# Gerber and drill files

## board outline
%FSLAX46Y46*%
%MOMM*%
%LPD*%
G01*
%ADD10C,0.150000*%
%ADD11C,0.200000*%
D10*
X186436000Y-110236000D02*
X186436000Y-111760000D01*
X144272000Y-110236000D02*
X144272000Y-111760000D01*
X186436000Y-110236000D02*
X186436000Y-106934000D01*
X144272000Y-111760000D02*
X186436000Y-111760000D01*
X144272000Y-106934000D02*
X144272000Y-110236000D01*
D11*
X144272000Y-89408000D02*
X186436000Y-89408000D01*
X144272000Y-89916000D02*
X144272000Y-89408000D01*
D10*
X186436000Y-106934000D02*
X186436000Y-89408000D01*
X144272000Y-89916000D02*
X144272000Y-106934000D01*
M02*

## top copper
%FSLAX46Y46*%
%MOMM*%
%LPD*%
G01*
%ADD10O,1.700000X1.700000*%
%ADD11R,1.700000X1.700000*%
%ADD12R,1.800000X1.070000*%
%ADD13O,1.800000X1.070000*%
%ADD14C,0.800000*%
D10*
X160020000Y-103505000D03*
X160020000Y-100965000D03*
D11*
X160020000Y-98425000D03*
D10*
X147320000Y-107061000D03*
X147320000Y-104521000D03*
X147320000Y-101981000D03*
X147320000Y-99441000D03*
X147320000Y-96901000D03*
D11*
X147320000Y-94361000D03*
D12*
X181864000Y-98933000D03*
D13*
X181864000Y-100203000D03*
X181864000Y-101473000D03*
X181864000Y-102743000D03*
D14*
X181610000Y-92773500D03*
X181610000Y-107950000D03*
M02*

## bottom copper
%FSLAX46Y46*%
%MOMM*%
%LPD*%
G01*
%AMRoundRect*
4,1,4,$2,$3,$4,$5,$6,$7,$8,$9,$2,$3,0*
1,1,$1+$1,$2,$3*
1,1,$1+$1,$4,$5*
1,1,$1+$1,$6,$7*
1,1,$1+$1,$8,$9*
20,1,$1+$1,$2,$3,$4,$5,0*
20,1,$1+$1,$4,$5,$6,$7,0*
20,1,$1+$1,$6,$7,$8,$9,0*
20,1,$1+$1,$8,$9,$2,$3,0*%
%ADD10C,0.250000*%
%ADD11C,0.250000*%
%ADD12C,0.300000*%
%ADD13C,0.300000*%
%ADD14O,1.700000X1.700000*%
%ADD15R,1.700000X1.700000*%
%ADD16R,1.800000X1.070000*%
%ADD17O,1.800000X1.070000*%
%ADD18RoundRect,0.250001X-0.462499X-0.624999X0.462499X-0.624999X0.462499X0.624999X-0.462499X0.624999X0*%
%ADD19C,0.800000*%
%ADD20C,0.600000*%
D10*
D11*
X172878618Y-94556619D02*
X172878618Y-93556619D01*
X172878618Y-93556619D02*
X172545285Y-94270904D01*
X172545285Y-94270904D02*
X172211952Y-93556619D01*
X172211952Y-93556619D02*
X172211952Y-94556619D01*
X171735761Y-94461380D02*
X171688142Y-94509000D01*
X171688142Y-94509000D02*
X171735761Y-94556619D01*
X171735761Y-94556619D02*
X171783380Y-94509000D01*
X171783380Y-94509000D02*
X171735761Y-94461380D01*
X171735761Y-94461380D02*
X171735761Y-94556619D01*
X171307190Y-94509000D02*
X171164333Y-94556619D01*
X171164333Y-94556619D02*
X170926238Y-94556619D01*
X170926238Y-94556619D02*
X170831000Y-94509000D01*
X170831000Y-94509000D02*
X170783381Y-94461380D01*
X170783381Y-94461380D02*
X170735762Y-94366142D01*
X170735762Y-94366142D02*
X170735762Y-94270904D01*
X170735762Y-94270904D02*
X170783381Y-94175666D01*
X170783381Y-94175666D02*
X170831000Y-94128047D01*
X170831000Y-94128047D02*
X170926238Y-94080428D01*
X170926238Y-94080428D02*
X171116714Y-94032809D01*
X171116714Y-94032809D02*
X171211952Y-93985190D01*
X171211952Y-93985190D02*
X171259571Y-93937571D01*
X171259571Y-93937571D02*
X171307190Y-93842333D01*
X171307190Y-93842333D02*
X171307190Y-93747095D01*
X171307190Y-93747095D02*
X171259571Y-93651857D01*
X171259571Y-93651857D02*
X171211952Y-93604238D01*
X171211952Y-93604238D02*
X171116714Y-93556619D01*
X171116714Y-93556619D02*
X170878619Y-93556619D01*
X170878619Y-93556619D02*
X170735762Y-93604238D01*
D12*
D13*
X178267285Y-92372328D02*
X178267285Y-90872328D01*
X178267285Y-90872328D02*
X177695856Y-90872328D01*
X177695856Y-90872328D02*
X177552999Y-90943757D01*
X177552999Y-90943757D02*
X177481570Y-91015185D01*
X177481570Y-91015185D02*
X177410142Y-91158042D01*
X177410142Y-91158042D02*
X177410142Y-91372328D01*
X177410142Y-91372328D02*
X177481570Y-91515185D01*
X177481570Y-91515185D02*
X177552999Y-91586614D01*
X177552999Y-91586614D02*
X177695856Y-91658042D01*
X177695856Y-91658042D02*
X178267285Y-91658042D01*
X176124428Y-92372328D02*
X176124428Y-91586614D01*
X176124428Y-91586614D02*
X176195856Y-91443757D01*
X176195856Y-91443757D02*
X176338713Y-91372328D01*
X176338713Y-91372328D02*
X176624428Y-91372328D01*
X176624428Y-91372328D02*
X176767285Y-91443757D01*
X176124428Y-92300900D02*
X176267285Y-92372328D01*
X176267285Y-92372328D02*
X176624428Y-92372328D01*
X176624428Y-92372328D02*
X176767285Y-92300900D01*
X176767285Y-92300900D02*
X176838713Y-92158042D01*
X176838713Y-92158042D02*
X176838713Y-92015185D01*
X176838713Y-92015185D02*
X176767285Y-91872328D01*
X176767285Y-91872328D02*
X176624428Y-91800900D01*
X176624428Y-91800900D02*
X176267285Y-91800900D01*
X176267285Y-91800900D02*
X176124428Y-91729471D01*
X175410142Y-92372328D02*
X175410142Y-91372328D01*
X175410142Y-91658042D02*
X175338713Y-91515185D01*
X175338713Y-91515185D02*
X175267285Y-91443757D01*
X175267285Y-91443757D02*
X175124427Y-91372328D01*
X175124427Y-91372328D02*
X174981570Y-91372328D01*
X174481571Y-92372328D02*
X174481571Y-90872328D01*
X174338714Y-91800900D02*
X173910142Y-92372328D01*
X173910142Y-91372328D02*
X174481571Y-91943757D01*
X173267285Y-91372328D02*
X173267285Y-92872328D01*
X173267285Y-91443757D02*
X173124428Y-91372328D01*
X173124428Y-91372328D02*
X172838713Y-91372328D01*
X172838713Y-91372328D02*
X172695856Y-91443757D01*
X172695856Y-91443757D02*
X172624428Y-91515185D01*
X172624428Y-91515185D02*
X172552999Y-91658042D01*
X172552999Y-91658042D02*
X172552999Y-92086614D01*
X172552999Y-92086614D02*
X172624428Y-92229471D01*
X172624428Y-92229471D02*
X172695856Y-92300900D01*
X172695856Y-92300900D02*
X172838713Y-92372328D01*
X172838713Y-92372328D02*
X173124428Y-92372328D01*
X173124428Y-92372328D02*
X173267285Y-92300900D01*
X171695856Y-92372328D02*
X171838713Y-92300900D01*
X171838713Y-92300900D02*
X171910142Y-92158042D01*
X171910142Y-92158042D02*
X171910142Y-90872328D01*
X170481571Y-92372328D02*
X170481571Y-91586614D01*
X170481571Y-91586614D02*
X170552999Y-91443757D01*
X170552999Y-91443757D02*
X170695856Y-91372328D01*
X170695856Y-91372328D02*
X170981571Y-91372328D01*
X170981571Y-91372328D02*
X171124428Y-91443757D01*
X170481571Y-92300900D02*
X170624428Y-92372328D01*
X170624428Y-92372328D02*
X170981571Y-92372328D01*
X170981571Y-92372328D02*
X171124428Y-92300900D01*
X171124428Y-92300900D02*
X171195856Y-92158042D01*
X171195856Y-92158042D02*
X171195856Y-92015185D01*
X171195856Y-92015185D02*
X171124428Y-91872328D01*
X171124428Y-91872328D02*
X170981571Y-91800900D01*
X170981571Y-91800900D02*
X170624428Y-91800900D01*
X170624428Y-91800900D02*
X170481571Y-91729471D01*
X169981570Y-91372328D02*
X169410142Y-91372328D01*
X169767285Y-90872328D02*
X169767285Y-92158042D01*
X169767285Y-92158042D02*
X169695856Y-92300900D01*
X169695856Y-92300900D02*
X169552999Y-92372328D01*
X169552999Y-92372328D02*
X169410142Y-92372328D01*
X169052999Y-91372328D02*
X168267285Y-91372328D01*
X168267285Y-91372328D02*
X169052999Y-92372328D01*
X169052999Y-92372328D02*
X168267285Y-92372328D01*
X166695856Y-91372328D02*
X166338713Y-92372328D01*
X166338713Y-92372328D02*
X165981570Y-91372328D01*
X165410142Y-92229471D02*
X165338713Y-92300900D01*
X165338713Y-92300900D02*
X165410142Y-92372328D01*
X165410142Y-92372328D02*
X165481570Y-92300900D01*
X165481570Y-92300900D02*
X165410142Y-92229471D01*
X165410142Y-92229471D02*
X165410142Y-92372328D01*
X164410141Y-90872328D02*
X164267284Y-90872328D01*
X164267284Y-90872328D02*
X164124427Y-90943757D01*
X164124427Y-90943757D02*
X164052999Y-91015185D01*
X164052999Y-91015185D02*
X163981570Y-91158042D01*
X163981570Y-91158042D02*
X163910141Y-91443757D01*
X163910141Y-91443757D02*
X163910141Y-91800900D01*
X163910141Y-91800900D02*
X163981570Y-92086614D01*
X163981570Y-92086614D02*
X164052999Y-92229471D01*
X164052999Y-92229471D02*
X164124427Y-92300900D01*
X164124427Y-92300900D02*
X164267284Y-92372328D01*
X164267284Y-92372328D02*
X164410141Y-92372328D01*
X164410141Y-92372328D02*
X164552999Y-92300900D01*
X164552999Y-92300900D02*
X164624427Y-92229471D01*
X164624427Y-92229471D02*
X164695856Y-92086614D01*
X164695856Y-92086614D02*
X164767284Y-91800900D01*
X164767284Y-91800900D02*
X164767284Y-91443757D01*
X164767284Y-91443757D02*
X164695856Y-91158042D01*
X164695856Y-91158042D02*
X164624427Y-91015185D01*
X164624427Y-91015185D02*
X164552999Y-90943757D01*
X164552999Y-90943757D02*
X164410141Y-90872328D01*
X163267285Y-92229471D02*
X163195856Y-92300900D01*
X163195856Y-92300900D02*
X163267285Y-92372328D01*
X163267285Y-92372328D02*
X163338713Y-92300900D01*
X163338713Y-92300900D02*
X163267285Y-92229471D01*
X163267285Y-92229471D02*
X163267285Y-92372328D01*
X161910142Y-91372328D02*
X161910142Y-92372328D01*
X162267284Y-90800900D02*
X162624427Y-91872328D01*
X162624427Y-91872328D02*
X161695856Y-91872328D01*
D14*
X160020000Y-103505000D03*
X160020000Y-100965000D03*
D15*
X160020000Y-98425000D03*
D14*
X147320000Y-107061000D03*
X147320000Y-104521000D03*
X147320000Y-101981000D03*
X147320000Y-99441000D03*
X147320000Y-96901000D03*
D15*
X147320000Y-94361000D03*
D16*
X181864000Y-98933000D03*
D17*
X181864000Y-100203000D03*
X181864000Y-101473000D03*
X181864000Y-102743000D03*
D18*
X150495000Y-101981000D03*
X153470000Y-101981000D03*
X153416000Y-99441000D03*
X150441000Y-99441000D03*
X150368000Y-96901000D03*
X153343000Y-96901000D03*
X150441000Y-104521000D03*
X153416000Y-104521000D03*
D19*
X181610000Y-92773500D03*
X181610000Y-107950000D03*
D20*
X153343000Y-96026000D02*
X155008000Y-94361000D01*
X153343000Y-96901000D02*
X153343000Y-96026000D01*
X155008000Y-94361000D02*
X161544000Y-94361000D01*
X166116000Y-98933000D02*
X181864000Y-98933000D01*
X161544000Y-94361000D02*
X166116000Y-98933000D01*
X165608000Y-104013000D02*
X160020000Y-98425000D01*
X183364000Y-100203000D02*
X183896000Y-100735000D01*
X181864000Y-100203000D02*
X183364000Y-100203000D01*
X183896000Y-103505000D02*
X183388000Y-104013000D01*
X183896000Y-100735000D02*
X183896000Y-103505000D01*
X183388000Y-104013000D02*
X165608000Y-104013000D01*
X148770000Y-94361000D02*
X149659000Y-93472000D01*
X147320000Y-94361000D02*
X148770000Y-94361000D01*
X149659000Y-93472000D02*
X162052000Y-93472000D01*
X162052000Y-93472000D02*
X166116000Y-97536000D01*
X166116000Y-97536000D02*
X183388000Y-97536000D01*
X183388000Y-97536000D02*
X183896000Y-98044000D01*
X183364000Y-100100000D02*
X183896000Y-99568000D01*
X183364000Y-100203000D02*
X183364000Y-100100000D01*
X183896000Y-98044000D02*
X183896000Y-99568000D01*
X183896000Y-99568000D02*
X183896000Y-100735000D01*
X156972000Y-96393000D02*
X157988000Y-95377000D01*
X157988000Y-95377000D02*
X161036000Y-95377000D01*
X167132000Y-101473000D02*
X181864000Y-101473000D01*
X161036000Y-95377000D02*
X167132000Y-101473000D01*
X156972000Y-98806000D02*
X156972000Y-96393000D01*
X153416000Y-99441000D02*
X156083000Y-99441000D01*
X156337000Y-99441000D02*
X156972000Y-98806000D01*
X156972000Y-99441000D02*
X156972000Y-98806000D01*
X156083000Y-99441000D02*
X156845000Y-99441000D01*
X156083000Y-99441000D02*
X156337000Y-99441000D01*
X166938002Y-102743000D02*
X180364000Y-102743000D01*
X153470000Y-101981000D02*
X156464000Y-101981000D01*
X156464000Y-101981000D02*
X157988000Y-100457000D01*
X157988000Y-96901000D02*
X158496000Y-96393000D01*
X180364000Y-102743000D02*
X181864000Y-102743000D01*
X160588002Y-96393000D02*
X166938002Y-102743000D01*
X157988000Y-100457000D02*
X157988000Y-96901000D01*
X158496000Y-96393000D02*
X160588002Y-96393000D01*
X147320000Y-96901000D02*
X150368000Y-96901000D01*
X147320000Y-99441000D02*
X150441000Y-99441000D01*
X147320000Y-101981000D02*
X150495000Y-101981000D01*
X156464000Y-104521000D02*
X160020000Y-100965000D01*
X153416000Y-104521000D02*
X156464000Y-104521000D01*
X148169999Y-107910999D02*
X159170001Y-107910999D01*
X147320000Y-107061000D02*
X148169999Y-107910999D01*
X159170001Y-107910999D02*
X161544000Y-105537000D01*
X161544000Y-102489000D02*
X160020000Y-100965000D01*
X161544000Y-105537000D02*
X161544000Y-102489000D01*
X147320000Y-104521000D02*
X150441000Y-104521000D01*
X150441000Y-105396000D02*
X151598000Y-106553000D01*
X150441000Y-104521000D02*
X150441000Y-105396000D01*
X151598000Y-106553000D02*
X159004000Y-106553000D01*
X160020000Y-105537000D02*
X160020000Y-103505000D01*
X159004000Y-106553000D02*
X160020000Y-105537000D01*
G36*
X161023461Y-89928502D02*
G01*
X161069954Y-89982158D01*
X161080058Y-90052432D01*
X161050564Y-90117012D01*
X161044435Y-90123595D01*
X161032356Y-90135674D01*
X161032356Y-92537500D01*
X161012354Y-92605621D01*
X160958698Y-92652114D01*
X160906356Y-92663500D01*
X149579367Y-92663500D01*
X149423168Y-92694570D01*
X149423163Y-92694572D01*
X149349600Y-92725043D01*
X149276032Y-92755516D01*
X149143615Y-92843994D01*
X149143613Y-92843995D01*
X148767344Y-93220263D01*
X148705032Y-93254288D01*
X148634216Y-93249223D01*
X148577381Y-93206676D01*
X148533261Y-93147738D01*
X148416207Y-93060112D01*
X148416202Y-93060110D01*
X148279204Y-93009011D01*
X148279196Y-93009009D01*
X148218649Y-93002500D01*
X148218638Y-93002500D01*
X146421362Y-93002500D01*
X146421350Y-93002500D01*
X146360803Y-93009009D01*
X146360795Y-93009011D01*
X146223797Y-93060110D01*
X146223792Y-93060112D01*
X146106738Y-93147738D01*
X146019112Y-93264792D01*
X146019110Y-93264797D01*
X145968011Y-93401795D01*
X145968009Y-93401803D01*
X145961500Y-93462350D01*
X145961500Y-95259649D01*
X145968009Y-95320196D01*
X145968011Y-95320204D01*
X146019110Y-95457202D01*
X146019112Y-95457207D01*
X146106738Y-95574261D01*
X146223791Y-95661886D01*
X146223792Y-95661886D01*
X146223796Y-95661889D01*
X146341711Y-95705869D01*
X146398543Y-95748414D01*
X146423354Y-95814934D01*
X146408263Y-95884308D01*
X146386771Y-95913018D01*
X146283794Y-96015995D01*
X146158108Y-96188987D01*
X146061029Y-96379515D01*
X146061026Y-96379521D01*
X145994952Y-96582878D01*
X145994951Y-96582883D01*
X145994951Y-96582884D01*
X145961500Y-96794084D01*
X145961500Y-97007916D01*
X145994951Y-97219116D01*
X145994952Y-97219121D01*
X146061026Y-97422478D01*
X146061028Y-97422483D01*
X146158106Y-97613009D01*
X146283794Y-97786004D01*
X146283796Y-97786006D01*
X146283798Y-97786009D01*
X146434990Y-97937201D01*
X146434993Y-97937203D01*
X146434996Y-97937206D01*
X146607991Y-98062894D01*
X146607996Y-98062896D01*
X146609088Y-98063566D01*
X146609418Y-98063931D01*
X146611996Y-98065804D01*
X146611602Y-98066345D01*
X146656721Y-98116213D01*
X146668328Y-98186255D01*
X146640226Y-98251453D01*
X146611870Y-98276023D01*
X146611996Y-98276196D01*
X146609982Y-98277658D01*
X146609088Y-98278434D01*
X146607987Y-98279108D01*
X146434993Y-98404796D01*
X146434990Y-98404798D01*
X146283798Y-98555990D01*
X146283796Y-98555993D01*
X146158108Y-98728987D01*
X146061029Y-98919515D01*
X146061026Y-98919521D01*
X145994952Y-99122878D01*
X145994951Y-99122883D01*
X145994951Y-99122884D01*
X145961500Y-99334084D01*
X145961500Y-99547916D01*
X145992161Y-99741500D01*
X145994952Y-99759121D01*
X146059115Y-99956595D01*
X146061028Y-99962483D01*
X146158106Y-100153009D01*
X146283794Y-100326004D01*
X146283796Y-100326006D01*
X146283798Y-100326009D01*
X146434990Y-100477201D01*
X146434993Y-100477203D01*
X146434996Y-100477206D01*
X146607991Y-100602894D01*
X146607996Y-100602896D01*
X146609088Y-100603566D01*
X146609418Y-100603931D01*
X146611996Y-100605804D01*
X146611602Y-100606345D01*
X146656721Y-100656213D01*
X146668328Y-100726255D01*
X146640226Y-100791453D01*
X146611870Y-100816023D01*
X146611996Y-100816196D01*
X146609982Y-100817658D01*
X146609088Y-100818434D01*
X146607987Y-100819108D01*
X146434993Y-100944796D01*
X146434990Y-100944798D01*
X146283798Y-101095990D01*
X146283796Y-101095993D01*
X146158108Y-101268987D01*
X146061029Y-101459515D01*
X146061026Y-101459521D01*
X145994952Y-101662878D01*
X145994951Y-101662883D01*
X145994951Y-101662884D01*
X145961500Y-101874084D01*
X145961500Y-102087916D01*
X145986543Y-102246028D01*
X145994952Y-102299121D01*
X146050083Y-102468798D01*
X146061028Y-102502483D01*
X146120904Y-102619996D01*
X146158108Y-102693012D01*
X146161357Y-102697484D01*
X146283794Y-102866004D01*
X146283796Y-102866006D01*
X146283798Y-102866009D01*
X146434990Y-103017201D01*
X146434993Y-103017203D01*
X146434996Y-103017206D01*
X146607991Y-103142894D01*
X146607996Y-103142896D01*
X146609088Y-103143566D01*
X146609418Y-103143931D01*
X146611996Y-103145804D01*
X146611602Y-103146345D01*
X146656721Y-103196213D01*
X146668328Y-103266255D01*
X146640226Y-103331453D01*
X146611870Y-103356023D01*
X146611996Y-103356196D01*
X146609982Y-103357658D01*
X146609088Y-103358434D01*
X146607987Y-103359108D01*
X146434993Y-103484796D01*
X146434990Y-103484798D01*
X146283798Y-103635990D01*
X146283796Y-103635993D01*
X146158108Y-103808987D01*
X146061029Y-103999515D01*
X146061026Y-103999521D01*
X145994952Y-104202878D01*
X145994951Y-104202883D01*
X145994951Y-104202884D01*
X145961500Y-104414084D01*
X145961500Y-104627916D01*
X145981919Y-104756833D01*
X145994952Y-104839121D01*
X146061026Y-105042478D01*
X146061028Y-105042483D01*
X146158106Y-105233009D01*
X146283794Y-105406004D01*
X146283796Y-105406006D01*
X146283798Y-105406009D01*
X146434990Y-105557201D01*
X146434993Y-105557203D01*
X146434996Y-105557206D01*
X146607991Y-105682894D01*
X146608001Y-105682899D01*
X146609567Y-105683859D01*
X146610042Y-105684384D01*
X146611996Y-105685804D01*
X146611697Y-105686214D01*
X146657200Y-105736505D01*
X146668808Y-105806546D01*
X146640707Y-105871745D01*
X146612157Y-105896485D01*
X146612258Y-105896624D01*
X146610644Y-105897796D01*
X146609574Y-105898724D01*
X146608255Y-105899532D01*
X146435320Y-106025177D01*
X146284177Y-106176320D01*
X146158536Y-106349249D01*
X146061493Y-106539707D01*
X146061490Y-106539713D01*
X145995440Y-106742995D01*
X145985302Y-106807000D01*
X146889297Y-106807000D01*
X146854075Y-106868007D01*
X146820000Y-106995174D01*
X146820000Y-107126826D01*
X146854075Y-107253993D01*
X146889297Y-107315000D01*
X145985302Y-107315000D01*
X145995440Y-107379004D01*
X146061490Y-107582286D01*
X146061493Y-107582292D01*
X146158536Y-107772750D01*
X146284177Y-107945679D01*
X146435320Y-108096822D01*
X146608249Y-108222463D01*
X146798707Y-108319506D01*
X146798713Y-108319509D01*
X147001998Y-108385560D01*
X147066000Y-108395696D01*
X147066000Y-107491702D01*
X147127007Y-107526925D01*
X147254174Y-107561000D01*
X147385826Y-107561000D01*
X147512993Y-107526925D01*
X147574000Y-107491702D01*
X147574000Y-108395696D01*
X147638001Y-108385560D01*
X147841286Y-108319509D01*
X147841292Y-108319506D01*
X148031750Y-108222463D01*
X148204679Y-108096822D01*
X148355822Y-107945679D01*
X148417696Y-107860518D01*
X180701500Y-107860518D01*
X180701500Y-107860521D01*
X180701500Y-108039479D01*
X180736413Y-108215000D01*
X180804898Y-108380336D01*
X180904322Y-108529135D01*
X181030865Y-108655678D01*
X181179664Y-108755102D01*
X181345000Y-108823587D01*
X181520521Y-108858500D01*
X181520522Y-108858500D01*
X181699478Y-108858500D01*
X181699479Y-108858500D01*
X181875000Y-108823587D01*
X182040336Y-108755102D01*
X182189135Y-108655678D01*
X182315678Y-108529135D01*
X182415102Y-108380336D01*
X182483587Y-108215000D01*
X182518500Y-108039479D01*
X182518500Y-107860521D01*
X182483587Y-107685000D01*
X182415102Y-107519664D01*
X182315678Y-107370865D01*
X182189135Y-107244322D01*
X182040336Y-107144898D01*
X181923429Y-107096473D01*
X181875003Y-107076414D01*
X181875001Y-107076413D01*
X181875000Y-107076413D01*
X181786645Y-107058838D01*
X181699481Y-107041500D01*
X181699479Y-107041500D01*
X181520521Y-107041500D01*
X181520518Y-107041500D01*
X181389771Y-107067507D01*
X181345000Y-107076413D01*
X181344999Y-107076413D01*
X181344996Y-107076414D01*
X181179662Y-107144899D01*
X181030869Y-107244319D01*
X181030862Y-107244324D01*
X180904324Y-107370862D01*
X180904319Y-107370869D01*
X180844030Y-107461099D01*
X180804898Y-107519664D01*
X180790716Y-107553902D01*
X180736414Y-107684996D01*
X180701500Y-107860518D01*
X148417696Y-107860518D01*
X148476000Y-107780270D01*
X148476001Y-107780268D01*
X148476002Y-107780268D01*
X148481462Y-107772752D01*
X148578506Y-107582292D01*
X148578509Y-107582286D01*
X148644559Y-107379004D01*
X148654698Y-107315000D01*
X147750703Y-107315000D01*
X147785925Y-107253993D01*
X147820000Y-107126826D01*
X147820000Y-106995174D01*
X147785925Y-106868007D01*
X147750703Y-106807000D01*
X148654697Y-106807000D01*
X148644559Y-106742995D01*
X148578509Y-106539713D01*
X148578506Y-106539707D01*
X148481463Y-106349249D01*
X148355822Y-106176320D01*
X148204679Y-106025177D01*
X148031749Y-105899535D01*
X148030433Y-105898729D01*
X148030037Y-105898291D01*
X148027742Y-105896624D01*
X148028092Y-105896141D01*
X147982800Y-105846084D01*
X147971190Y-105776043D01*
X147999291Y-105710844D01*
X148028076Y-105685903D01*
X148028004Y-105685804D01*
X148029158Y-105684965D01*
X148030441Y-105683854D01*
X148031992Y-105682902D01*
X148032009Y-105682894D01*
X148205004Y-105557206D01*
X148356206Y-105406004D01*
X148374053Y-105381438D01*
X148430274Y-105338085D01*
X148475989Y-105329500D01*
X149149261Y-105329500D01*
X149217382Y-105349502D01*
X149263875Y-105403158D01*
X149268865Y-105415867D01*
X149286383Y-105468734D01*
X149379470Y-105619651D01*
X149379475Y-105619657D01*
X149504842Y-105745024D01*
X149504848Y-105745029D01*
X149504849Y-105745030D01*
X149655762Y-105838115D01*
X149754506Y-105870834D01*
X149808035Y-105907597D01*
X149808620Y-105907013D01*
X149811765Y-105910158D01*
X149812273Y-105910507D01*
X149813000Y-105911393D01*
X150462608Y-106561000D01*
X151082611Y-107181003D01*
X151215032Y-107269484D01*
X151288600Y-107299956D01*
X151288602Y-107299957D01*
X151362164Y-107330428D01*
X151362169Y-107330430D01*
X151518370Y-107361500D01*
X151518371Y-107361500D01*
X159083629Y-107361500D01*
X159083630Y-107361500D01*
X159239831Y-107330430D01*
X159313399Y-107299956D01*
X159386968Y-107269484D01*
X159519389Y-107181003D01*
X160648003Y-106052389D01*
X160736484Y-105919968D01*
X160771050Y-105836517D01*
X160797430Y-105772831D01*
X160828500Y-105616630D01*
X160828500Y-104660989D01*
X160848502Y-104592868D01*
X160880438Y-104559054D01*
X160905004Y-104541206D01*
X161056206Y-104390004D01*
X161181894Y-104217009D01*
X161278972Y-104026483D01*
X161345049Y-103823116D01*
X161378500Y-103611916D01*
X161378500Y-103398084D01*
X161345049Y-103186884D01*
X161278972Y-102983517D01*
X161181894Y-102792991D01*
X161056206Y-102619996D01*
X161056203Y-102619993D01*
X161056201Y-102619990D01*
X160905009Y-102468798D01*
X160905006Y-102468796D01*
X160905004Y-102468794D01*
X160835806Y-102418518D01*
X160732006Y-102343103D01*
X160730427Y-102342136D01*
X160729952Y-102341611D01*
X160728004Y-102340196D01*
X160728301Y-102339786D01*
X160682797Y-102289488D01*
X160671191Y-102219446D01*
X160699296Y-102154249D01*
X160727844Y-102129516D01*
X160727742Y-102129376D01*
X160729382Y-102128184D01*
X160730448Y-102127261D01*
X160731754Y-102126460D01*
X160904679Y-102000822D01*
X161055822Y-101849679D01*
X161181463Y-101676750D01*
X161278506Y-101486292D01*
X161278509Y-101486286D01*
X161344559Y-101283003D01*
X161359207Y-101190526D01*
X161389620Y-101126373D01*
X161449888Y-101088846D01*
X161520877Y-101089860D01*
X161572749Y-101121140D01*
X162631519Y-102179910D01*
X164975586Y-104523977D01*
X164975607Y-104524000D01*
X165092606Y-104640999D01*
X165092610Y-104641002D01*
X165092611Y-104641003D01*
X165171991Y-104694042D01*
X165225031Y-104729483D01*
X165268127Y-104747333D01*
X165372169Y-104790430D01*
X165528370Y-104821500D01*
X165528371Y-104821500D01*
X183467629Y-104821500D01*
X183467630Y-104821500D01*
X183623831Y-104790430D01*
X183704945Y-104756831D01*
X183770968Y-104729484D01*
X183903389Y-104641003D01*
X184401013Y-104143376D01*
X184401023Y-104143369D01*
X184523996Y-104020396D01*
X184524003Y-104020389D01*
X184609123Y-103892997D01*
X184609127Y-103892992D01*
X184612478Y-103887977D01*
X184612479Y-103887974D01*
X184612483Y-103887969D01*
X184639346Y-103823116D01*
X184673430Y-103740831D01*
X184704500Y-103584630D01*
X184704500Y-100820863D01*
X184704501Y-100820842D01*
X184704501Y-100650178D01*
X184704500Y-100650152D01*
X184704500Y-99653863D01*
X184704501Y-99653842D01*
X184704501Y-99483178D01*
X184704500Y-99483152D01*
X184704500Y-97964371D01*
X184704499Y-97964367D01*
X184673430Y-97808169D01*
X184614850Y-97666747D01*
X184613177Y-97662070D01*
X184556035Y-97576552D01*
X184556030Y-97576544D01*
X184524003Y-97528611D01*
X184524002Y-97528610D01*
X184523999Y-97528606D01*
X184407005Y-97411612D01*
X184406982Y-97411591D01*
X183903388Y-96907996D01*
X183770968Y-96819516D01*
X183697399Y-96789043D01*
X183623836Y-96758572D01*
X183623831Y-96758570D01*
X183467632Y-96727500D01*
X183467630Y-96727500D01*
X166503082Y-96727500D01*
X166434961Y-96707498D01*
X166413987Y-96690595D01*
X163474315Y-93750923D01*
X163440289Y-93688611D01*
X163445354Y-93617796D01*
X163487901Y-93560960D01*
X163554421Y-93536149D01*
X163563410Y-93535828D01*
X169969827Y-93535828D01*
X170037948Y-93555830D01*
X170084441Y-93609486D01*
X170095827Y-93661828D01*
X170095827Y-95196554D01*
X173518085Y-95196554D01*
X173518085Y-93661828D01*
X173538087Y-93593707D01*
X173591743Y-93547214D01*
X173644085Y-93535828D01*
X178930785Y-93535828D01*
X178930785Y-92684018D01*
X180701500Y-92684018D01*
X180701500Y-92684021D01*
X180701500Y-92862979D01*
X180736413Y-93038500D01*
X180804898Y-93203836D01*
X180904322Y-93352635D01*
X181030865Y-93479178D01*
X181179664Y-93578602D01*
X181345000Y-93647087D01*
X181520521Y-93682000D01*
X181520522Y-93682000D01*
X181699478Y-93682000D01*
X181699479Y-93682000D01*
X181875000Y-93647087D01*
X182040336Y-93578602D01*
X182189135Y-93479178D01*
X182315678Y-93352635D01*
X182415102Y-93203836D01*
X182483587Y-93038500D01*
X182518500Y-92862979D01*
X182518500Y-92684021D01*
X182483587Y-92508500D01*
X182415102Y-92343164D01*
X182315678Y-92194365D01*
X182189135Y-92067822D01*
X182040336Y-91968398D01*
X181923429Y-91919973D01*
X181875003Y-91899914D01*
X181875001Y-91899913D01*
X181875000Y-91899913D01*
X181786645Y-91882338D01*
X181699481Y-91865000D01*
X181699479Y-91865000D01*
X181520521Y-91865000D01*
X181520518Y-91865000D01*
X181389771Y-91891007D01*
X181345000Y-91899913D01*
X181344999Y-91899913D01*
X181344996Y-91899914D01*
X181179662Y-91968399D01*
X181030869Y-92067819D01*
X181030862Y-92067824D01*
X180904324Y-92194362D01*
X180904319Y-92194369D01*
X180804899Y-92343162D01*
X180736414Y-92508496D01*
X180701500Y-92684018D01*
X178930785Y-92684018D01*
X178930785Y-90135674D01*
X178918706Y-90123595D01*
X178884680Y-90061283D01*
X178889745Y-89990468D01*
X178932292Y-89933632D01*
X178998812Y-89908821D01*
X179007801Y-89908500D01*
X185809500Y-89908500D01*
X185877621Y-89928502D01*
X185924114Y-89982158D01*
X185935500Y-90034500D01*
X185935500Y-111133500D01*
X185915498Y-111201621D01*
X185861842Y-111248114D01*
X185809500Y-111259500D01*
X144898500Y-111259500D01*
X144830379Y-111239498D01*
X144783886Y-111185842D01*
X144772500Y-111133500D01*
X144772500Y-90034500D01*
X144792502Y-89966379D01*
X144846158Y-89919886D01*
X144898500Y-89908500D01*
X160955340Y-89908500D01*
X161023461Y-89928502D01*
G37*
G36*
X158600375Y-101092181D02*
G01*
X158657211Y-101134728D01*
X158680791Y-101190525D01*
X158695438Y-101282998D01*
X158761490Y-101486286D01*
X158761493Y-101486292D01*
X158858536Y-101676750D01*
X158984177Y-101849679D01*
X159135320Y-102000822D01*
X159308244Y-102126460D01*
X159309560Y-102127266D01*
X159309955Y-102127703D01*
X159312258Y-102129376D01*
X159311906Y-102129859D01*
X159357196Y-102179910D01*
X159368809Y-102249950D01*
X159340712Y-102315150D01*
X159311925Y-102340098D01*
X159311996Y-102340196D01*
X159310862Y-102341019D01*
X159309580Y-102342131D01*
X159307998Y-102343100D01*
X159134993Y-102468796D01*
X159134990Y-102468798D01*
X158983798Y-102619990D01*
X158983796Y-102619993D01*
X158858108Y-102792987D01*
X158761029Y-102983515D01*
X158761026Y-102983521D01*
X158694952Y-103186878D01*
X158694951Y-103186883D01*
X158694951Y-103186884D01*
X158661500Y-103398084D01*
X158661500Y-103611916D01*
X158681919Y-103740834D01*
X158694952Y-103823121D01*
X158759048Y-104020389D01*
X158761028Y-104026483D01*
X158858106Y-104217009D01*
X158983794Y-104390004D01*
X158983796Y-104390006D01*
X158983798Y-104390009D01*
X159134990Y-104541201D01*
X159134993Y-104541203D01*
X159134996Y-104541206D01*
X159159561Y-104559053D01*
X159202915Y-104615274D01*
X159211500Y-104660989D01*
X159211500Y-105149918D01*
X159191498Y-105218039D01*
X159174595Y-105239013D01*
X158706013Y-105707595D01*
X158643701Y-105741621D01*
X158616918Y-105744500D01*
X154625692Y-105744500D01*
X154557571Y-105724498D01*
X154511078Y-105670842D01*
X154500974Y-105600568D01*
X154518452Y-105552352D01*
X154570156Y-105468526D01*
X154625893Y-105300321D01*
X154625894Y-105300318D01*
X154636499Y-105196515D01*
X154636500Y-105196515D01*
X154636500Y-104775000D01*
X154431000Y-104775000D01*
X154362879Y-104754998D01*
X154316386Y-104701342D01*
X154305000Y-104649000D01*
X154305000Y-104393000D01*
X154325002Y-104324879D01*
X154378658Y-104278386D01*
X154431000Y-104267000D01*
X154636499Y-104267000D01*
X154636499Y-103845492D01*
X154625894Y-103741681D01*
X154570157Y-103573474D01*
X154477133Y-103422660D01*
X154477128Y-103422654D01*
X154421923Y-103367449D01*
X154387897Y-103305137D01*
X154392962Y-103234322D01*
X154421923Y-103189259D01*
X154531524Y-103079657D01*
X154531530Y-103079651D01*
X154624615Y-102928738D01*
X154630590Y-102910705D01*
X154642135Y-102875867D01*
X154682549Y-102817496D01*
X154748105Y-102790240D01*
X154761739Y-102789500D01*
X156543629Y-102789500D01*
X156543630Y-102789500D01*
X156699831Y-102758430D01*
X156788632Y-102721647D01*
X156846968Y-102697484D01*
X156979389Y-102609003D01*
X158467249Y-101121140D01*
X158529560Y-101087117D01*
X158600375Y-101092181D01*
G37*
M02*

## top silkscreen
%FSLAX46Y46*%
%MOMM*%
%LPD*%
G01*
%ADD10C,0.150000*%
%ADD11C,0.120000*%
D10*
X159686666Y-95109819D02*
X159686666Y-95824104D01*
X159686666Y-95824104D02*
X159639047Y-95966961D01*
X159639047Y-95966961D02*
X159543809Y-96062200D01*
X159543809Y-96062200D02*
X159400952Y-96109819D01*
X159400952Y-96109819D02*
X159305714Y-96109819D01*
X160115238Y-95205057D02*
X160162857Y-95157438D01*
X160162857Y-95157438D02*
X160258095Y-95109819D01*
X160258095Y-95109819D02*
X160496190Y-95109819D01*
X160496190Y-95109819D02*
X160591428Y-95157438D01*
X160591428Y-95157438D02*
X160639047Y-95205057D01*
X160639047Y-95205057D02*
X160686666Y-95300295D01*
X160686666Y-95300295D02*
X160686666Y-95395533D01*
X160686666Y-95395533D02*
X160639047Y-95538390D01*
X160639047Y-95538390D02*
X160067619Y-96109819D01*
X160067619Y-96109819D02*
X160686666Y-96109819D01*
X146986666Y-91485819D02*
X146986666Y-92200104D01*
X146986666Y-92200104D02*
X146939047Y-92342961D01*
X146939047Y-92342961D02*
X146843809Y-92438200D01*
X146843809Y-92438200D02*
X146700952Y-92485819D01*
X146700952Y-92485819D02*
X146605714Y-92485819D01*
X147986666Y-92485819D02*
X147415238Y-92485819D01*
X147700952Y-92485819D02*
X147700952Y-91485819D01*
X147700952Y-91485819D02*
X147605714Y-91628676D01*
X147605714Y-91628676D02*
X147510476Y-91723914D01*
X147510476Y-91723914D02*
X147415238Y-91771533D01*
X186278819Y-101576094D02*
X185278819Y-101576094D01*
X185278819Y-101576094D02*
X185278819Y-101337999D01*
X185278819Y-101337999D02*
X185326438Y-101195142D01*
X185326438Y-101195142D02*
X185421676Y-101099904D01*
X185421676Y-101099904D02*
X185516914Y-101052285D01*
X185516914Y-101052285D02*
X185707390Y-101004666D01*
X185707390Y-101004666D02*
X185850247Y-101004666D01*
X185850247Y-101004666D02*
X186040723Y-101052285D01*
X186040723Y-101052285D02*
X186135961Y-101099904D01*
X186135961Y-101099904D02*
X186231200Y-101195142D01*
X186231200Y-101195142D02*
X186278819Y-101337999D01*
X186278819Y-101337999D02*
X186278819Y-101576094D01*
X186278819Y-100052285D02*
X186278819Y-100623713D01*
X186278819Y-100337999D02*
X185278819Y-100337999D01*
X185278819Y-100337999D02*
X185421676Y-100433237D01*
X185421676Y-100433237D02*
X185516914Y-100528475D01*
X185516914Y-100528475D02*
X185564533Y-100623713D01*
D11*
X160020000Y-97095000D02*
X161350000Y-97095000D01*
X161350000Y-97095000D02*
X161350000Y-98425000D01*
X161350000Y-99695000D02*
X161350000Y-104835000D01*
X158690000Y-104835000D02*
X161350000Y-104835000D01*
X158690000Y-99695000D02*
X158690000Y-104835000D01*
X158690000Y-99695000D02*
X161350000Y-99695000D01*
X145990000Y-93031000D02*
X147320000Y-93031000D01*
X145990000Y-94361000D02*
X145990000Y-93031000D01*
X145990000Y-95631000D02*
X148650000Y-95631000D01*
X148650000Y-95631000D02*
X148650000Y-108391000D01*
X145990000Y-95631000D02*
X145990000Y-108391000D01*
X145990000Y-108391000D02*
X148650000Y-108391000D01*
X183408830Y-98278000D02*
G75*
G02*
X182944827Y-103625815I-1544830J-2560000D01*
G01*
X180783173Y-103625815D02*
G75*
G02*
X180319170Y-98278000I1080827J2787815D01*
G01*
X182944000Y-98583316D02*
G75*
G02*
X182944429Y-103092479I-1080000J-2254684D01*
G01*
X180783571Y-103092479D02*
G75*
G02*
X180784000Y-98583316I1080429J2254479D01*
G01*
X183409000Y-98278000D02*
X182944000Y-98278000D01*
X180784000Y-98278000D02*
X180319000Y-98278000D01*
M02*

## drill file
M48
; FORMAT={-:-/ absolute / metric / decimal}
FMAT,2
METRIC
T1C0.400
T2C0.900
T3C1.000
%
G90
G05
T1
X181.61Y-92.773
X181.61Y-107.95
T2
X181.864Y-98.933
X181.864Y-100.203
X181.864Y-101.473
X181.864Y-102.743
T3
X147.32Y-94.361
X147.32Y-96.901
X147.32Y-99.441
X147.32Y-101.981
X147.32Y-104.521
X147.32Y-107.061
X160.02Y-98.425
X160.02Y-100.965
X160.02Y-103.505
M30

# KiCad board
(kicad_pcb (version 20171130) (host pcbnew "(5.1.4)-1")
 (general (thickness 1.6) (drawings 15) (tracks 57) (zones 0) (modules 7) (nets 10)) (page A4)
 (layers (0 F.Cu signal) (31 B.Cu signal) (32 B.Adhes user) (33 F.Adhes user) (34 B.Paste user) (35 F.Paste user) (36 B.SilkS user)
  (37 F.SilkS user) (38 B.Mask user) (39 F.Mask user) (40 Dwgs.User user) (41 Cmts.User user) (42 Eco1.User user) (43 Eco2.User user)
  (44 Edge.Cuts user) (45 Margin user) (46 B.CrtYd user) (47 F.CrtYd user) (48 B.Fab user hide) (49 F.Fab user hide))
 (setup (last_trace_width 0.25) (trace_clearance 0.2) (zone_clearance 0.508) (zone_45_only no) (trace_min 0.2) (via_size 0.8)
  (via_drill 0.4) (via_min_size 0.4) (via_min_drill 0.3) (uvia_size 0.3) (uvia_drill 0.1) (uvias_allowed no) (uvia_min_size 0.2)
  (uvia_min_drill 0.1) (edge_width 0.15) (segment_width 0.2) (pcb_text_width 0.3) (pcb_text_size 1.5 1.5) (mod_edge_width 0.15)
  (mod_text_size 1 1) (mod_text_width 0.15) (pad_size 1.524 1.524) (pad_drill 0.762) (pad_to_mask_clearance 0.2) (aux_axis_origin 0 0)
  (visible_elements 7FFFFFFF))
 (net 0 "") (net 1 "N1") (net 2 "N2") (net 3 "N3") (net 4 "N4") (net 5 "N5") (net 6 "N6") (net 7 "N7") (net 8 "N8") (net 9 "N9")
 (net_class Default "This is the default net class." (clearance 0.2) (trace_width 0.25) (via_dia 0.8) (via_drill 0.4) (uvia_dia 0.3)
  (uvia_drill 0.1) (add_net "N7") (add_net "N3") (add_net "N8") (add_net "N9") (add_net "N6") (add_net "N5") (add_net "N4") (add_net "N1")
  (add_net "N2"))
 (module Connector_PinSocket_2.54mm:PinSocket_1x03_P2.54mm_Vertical (layer F.Cu) (at 160.02 98.425)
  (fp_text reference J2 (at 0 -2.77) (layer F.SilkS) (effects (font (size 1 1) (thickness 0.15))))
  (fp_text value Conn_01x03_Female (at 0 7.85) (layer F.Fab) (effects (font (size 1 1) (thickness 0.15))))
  (fp_line (start 0 -1.33) (end 1.33 -1.33) (layer F.SilkS) (width 0.12))
  (fp_line (start 1.33 -1.33) (end 1.33 0) (layer F.SilkS) (width 0.12))
  (fp_line (start 1.33 1.27) (end 1.33 6.41) (layer F.SilkS) (width 0.12))
  (fp_line (start -1.33 6.41) (end 1.33 6.41) (layer F.SilkS) (width 0.12))
  (fp_line (start -1.33 1.27) (end -1.33 6.41) (layer F.SilkS) (width 0.12))
  (fp_line (start -1.33 1.27) (end 1.33 1.27) (layer F.SilkS) (width 0.12))
  (pad 3 thru_hole oval (at 0 5.08) (size 1.7 1.7) (drill 1) (layers *.Cu *.Mask) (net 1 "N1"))
  (pad 2 thru_hole oval (at 0 2.54) (size 1.7 1.7) (drill 1) (layers *.Cu *.Mask) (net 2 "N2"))
  (pad 1 thru_hole rect (at 0 0) (size 1.7 1.7) (drill 1) (layers *.Cu *.Mask) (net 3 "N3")))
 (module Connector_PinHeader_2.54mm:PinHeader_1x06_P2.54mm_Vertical (layer F.Cu) (at 147.32 94.361)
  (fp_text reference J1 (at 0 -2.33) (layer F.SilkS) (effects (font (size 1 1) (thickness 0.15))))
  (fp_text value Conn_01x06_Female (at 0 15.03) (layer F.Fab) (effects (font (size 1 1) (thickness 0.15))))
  (fp_line (start -1.33 -1.33) (end 0 -1.33) (layer F.SilkS) (width 0.12))
  (fp_line (start -1.33 0) (end -1.33 -1.33) (layer F.SilkS) (width 0.12))
  (fp_line (start -1.33 1.27) (end 1.33 1.27) (layer F.SilkS) (width 0.12))
  (fp_line (start 1.33 1.27) (end 1.33 14.03) (layer F.SilkS) (width 0.12))
  (fp_line (start -1.33 1.27) (end -1.33 14.03) (layer F.SilkS) (width 0.12))
  (fp_line (start -1.33 14.03) (end 1.33 14.03) (layer F.SilkS) (width 0.12))
  (pad 6 thru_hole oval (at 0 12.7) (size 1.7 1.7) (drill 1) (layers *.Cu *.Mask) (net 2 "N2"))
  (pad 5 thru_hole oval (at 0 10.16) (size 1.7 1.7) (drill 1) (layers *.Cu *.Mask) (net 1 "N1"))
  (pad 4 thru_hole oval (at 0 7.62) (size 1.7 1.7) (drill 1) (layers *.Cu *.Mask) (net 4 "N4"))
  (pad 3 thru_hole oval (at 0 5.08) (size 1.7 1.7) (drill 1) (layers *.Cu *.Mask) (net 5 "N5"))
  (pad 2 thru_hole oval (at 0 2.54) (size 1.7 1.7) (drill 1) (layers *.Cu *.Mask) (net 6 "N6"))
  (pad 1 thru_hole rect (at 0 0) (size 1.7 1.7) (drill 1) (layers *.Cu *.Mask) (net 3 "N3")))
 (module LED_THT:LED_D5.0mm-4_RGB (layer F.Cu) (at 181.864 98.933 270)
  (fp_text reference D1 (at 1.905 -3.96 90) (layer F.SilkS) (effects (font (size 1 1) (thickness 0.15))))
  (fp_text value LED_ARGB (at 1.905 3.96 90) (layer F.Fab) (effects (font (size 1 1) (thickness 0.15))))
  (fp_arc (start 1.905 0) (end -0.655 -1.54483) (angle 127.7) (layer F.SilkS) (width 0.12))
  (fp_arc (start 1.905 0) (end -0.655 1.54483) (angle -127.7) (layer F.SilkS) (width 0.12))
  (fp_arc (start 1.905 0) (end -0.349684 -1.08) (angle 128.8) (layer F.SilkS) (width 0.12))
  (fp_arc (start 1.905 0) (end -0.349684 1.08) (angle -128.8) (layer F.SilkS) (width 0.12))
  (fp_line (start -0.655 -1.545) (end -0.655 -1.08) (layer F.SilkS) (width 0.12))
  (fp_line (start -0.655 1.08) (end -0.655 1.545) (layer F.SilkS) (width 0.12))
  (pad 1 thru_hole rect (at 0 0 270) (size 1.07 1.8) (drill 0.9) (layers *.Cu *.Mask) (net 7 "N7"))
  (pad 2 thru_hole oval (at 1.27 0 270) (size 1.07 1.8) (drill 0.9) (layers *.Cu *.Mask) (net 3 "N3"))
  (pad 3 thru_hole oval (at 2.54 0 270) (size 1.07 1.8) (drill 0.9) (layers *.Cu *.Mask) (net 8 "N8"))
  (pad 4 thru_hole oval (at 3.81 0 270) (size 1.07 1.8) (drill 0.9) (layers *.Cu *.Mask) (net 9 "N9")))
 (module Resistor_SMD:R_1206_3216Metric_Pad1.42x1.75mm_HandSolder (layer B.Cu) (at 151.9825 101.981)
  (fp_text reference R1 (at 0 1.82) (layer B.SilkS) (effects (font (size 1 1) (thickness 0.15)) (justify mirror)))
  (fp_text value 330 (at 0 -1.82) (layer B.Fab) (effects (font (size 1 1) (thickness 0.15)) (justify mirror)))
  (pad 1 smd roundrect (at -1.4875 0) (size 1.425 1.75) (layers B.Cu B.Paste B.Mask) (roundrect_rratio 0.175439) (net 4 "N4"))
  (pad 2 smd roundrect (at 1.4875 0) (size 1.425 1.75) (layers B.Cu B.Paste B.Mask) (roundrect_rratio 0.175439) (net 9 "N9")))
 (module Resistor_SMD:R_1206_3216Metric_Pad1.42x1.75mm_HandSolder (layer B.Cu) (at 151.9285 99.441)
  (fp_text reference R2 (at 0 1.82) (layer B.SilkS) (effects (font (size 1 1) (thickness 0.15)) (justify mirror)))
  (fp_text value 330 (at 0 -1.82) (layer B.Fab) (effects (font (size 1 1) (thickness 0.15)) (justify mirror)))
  (pad 2 smd roundrect (at 1.4875 0) (size 1.425 1.75) (layers B.Cu B.Paste B.Mask) (roundrect_rratio 0.175439) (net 8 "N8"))
  (pad 1 smd roundrect (at -1.4875 0) (size 1.425 1.75) (layers B.Cu B.Paste B.Mask) (roundrect_rratio 0.175439) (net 5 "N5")))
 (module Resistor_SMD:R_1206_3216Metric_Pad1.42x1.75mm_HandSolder (layer B.Cu) (at 151.8555 96.901)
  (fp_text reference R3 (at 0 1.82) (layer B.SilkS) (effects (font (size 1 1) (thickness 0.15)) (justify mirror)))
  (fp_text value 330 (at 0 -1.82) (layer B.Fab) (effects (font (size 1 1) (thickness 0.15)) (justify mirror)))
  (pad 1 smd roundrect (at -1.4875 0) (size 1.425 1.75) (layers B.Cu B.Paste B.Mask) (roundrect_rratio 0.175439) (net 6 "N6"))
  (pad 2 smd roundrect (at 1.4875 0) (size 1.425 1.75) (layers B.Cu B.Paste B.Mask) (roundrect_rratio 0.175439) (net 7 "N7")))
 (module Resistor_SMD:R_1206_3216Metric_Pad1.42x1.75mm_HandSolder (layer B.Cu) (at 151.9285 104.521)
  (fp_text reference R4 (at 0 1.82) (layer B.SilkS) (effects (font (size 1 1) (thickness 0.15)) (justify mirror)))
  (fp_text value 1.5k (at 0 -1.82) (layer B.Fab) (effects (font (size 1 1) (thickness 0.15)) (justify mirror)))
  (pad 1 smd roundrect (at -1.4875 0) (size 1.425 1.75) (layers B.Cu B.Paste B.Mask) (roundrect_rratio 0.175439) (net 1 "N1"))
  (pad 2 smd roundrect (at 1.4875 0) (size 1.425 1.75) (layers B.Cu B.Paste B.Mask) (roundrect_rratio 0.175439) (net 2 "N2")))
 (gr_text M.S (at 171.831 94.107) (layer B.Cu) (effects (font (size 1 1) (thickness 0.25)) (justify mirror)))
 (gr_line (start 186.436 110.236) (end 186.436 111.76) (layer Edge.Cuts) (width 0.15))
 (gr_line (start 144.272 110.236) (end 144.272 111.76) (layer Edge.Cuts) (width 0.15))
 (gr_line (start 186.436 110.236) (end 186.436 106.934) (layer Edge.Cuts) (width 0.15))
 (gr_line (start 144.272 111.76) (end 186.436 111.76) (layer Edge.Cuts) (width 0.15))
 (gr_line (start 144.272 106.934) (end 144.272 110.236) (layer Edge.Cuts) (width 0.15))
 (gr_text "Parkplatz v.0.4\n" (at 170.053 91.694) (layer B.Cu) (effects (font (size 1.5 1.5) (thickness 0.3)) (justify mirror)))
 (gr_line (start 144.272 89.408) (end 186.436 89.408) (layer Edge.Cuts) (width 0.2))
 (gr_line (start 144.272 89.916) (end 144.272 89.408) (layer Edge.Cuts) (width 0.2))
 (gr_line (start 186.436 106.934) (end 186.436 89.408) (layer Edge.Cuts) (width 0.15))
 (gr_line (start 144.272 89.916) (end 144.272 106.934) (layer Edge.Cuts) (width 0.15))
 (via (at 181.61 92.7735) (size 0.8) (drill 0.4) (layers F.Cu B.Cu) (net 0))
 (via (at 181.61 107.95) (size 0.8) (drill 0.4) (layers F.Cu B.Cu) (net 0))
 (segment (start 153.343 96.026) (end 155.008 94.361) (width 0.6) (layer B.Cu) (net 7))
 (segment (start 153.343 96.901) (end 153.343 96.026) (width 0.6) (layer B.Cu) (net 7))
 (segment (start 155.008 94.361) (end 161.544 94.361) (width 0.6) (layer B.Cu) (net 7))
 (segment (start 166.116 98.933) (end 181.864 98.933) (width 0.6) (layer B.Cu) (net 7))
 (segment (start 161.544 94.361) (end 166.116 98.933) (width 0.6) (layer B.Cu) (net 7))
 (segment (start 165.608 104.013) (end 160.02 98.425) (width 0.6) (layer B.Cu) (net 3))
 (segment (start 183.364 100.203) (end 183.896 100.735) (width 0.6) (layer B.Cu) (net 3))
 (segment (start 181.864 100.203) (end 183.364 100.203) (width 0.6) (layer B.Cu) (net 3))
 (segment (start 183.896 103.505) (end 183.388 104.013) (width 0.6) (layer B.Cu) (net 3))
 (segment (start 183.896 100.735) (end 183.896 103.505) (width 0.6) (layer B.Cu) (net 3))
 (segment (start 183.388 104.013) (end 165.608 104.013) (width 0.6) (layer B.Cu) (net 3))
 (segment (start 148.77 94.361) (end 149.659 93.472) (width 0.6) (layer B.Cu) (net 3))
 (segment (start 147.32 94.361) (end 148.77 94.361) (width 0.6) (layer B.Cu) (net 3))
 (segment (start 149.659 93.472) (end 162.052 93.472) (width 0.6) (layer B.Cu) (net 3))
 (segment (start 162.052 93.472) (end 166.116 97.536) (width 0.6) (layer B.Cu) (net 3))
 (segment (start 166.116 97.536) (end 183.388 97.536) (width 0.6) (layer B.Cu) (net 3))
 (segment (start 183.388 97.536) (end 183.896 98.044) (width 0.6) (layer B.Cu) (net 3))
 (segment (start 183.364 100.1) (end 183.896 99.568) (width 0.6) (layer B.Cu) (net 3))
 (segment (start 183.364 100.203) (end 183.364 100.1) (width 0.6) (layer B.Cu) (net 3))
 (segment (start 183.896 98.044) (end 183.896 99.568) (width 0.6) (layer B.Cu) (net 3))
 (segment (start 183.896 99.568) (end 183.896 100.735) (width 0.6) (layer B.Cu) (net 3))
 (segment (start 156.972 96.393) (end 157.988 95.377) (width 0.6) (layer B.Cu) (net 8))
 (segment (start 157.988 95.377) (end 161.036 95.377) (width 0.6) (layer B.Cu) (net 8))
 (segment (start 167.132 101.473) (end 181.864 101.473) (width 0.6) (layer B.Cu) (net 8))
 (segment (start 161.036 95.377) (end 167.132 101.473) (width 0.6) (layer B.Cu) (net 8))
 (segment (start 156.972 98.806) (end 156.972 96.393) (width 0.6) (layer B.Cu) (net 8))
 (segment (start 153.416 99.441) (end 156.083 99.441) (width 0.6) (layer B.Cu) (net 8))
 (segment (start 156.337 99.441) (end 156.972 98.806) (width 0.6) (layer B.Cu) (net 8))
 (segment (start 156.972 99.441) (end 156.972 98.806) (width 0.6) (layer B.Cu) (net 8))
 (segment (start 156.083 99.441) (end 156.845 99.441) (width 0.6) (layer B.Cu) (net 8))
 (segment (start 156.083 99.441) (end 156.337 99.441) (width 0.6) (layer B.Cu) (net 8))
 (segment (start 166.938002 102.743) (end 180.364 102.743) (width 0.6) (layer B.Cu) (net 9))
 (segment (start 153.47 101.981) (end 156.464 101.981) (width 0.6) (layer B.Cu) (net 9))
 (segment (start 156.464 101.981) (end 157.988 100.457) (width 0.6) (layer B.Cu) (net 9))
 (segment (start 157.988 96.901) (end 158.496 96.393) (width 0.6) (layer B.Cu) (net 9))
 (segment (start 180.364 102.743) (end 181.864 102.743) (width 0.6) (layer B.Cu) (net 9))
 (segment (start 160.588002 96.393) (end 166.938002 102.743) (width 0.6) (layer B.Cu) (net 9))
 (segment (start 157.988 100.457) (end 157.988 96.901) (width 0.6) (layer B.Cu) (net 9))
 (segment (start 158.496 96.393) (end 160.588002 96.393) (width 0.6) (layer B.Cu) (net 9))
 (segment (start 147.32 96.901) (end 150.368 96.901) (width 0.6) (layer B.Cu) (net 6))
 (segment (start 147.32 99.441) (end 150.441 99.441) (width 0.6) (layer B.Cu) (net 5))
 (segment (start 147.32 101.981) (end 150.495 101.981) (width 0.6) (layer B.Cu) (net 4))
 (segment (start 156.464 104.521) (end 160.02 100.965) (width 0.6) (layer B.Cu) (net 2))
 (segment (start 153.416 104.521) (end 156.464 104.521) (width 0.6) (layer B.Cu) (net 2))
 (segment (start 148.169999 107.910999) (end 159.170001 107.910999) (width 0.6) (layer B.Cu) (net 2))
 (segment (start 147.32 107.061) (end 148.169999 107.910999) (width 0.6) (layer B.Cu) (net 2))
 (segment (start 159.170001 107.910999) (end 161.544 105.537) (width 0.6) (layer B.Cu) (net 2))
 (segment (start 161.544 102.489) (end 160.02 100.965) (width 0.6) (layer B.Cu) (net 2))
 (segment (start 161.544 105.537) (end 161.544 102.489) (width 0.6) (layer B.Cu) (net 2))
 (segment (start 147.32 104.521) (end 150.441 104.521) (width 0.6) (layer B.Cu) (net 1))
 (segment (start 150.441 105.396) (end 151.598 106.553) (width 0.6) (layer B.Cu) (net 1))
 (segment (start 150.441 104.521) (end 150.441 105.396) (width 0.6) (layer B.Cu) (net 1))
 (segment (start 151.598 106.553) (end 159.004 106.553) (width 0.6) (layer B.Cu) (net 1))
 (segment (start 160.02 105.537) (end 160.02 103.505) (width 0.6) (layer B.Cu) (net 1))
 (segment (start 159.004 106.553) (end 160.02 105.537) (width 0.6) (layer B.Cu) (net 1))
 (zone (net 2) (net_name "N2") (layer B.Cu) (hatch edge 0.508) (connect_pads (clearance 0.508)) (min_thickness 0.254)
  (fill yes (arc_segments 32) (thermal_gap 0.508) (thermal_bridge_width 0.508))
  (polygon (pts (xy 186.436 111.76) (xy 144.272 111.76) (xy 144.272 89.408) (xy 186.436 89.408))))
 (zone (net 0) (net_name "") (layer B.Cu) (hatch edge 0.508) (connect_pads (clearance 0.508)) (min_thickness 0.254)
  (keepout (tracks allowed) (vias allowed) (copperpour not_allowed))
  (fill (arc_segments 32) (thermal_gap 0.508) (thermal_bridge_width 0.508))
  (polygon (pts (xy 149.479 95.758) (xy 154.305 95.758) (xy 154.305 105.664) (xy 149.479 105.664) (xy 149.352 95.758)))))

